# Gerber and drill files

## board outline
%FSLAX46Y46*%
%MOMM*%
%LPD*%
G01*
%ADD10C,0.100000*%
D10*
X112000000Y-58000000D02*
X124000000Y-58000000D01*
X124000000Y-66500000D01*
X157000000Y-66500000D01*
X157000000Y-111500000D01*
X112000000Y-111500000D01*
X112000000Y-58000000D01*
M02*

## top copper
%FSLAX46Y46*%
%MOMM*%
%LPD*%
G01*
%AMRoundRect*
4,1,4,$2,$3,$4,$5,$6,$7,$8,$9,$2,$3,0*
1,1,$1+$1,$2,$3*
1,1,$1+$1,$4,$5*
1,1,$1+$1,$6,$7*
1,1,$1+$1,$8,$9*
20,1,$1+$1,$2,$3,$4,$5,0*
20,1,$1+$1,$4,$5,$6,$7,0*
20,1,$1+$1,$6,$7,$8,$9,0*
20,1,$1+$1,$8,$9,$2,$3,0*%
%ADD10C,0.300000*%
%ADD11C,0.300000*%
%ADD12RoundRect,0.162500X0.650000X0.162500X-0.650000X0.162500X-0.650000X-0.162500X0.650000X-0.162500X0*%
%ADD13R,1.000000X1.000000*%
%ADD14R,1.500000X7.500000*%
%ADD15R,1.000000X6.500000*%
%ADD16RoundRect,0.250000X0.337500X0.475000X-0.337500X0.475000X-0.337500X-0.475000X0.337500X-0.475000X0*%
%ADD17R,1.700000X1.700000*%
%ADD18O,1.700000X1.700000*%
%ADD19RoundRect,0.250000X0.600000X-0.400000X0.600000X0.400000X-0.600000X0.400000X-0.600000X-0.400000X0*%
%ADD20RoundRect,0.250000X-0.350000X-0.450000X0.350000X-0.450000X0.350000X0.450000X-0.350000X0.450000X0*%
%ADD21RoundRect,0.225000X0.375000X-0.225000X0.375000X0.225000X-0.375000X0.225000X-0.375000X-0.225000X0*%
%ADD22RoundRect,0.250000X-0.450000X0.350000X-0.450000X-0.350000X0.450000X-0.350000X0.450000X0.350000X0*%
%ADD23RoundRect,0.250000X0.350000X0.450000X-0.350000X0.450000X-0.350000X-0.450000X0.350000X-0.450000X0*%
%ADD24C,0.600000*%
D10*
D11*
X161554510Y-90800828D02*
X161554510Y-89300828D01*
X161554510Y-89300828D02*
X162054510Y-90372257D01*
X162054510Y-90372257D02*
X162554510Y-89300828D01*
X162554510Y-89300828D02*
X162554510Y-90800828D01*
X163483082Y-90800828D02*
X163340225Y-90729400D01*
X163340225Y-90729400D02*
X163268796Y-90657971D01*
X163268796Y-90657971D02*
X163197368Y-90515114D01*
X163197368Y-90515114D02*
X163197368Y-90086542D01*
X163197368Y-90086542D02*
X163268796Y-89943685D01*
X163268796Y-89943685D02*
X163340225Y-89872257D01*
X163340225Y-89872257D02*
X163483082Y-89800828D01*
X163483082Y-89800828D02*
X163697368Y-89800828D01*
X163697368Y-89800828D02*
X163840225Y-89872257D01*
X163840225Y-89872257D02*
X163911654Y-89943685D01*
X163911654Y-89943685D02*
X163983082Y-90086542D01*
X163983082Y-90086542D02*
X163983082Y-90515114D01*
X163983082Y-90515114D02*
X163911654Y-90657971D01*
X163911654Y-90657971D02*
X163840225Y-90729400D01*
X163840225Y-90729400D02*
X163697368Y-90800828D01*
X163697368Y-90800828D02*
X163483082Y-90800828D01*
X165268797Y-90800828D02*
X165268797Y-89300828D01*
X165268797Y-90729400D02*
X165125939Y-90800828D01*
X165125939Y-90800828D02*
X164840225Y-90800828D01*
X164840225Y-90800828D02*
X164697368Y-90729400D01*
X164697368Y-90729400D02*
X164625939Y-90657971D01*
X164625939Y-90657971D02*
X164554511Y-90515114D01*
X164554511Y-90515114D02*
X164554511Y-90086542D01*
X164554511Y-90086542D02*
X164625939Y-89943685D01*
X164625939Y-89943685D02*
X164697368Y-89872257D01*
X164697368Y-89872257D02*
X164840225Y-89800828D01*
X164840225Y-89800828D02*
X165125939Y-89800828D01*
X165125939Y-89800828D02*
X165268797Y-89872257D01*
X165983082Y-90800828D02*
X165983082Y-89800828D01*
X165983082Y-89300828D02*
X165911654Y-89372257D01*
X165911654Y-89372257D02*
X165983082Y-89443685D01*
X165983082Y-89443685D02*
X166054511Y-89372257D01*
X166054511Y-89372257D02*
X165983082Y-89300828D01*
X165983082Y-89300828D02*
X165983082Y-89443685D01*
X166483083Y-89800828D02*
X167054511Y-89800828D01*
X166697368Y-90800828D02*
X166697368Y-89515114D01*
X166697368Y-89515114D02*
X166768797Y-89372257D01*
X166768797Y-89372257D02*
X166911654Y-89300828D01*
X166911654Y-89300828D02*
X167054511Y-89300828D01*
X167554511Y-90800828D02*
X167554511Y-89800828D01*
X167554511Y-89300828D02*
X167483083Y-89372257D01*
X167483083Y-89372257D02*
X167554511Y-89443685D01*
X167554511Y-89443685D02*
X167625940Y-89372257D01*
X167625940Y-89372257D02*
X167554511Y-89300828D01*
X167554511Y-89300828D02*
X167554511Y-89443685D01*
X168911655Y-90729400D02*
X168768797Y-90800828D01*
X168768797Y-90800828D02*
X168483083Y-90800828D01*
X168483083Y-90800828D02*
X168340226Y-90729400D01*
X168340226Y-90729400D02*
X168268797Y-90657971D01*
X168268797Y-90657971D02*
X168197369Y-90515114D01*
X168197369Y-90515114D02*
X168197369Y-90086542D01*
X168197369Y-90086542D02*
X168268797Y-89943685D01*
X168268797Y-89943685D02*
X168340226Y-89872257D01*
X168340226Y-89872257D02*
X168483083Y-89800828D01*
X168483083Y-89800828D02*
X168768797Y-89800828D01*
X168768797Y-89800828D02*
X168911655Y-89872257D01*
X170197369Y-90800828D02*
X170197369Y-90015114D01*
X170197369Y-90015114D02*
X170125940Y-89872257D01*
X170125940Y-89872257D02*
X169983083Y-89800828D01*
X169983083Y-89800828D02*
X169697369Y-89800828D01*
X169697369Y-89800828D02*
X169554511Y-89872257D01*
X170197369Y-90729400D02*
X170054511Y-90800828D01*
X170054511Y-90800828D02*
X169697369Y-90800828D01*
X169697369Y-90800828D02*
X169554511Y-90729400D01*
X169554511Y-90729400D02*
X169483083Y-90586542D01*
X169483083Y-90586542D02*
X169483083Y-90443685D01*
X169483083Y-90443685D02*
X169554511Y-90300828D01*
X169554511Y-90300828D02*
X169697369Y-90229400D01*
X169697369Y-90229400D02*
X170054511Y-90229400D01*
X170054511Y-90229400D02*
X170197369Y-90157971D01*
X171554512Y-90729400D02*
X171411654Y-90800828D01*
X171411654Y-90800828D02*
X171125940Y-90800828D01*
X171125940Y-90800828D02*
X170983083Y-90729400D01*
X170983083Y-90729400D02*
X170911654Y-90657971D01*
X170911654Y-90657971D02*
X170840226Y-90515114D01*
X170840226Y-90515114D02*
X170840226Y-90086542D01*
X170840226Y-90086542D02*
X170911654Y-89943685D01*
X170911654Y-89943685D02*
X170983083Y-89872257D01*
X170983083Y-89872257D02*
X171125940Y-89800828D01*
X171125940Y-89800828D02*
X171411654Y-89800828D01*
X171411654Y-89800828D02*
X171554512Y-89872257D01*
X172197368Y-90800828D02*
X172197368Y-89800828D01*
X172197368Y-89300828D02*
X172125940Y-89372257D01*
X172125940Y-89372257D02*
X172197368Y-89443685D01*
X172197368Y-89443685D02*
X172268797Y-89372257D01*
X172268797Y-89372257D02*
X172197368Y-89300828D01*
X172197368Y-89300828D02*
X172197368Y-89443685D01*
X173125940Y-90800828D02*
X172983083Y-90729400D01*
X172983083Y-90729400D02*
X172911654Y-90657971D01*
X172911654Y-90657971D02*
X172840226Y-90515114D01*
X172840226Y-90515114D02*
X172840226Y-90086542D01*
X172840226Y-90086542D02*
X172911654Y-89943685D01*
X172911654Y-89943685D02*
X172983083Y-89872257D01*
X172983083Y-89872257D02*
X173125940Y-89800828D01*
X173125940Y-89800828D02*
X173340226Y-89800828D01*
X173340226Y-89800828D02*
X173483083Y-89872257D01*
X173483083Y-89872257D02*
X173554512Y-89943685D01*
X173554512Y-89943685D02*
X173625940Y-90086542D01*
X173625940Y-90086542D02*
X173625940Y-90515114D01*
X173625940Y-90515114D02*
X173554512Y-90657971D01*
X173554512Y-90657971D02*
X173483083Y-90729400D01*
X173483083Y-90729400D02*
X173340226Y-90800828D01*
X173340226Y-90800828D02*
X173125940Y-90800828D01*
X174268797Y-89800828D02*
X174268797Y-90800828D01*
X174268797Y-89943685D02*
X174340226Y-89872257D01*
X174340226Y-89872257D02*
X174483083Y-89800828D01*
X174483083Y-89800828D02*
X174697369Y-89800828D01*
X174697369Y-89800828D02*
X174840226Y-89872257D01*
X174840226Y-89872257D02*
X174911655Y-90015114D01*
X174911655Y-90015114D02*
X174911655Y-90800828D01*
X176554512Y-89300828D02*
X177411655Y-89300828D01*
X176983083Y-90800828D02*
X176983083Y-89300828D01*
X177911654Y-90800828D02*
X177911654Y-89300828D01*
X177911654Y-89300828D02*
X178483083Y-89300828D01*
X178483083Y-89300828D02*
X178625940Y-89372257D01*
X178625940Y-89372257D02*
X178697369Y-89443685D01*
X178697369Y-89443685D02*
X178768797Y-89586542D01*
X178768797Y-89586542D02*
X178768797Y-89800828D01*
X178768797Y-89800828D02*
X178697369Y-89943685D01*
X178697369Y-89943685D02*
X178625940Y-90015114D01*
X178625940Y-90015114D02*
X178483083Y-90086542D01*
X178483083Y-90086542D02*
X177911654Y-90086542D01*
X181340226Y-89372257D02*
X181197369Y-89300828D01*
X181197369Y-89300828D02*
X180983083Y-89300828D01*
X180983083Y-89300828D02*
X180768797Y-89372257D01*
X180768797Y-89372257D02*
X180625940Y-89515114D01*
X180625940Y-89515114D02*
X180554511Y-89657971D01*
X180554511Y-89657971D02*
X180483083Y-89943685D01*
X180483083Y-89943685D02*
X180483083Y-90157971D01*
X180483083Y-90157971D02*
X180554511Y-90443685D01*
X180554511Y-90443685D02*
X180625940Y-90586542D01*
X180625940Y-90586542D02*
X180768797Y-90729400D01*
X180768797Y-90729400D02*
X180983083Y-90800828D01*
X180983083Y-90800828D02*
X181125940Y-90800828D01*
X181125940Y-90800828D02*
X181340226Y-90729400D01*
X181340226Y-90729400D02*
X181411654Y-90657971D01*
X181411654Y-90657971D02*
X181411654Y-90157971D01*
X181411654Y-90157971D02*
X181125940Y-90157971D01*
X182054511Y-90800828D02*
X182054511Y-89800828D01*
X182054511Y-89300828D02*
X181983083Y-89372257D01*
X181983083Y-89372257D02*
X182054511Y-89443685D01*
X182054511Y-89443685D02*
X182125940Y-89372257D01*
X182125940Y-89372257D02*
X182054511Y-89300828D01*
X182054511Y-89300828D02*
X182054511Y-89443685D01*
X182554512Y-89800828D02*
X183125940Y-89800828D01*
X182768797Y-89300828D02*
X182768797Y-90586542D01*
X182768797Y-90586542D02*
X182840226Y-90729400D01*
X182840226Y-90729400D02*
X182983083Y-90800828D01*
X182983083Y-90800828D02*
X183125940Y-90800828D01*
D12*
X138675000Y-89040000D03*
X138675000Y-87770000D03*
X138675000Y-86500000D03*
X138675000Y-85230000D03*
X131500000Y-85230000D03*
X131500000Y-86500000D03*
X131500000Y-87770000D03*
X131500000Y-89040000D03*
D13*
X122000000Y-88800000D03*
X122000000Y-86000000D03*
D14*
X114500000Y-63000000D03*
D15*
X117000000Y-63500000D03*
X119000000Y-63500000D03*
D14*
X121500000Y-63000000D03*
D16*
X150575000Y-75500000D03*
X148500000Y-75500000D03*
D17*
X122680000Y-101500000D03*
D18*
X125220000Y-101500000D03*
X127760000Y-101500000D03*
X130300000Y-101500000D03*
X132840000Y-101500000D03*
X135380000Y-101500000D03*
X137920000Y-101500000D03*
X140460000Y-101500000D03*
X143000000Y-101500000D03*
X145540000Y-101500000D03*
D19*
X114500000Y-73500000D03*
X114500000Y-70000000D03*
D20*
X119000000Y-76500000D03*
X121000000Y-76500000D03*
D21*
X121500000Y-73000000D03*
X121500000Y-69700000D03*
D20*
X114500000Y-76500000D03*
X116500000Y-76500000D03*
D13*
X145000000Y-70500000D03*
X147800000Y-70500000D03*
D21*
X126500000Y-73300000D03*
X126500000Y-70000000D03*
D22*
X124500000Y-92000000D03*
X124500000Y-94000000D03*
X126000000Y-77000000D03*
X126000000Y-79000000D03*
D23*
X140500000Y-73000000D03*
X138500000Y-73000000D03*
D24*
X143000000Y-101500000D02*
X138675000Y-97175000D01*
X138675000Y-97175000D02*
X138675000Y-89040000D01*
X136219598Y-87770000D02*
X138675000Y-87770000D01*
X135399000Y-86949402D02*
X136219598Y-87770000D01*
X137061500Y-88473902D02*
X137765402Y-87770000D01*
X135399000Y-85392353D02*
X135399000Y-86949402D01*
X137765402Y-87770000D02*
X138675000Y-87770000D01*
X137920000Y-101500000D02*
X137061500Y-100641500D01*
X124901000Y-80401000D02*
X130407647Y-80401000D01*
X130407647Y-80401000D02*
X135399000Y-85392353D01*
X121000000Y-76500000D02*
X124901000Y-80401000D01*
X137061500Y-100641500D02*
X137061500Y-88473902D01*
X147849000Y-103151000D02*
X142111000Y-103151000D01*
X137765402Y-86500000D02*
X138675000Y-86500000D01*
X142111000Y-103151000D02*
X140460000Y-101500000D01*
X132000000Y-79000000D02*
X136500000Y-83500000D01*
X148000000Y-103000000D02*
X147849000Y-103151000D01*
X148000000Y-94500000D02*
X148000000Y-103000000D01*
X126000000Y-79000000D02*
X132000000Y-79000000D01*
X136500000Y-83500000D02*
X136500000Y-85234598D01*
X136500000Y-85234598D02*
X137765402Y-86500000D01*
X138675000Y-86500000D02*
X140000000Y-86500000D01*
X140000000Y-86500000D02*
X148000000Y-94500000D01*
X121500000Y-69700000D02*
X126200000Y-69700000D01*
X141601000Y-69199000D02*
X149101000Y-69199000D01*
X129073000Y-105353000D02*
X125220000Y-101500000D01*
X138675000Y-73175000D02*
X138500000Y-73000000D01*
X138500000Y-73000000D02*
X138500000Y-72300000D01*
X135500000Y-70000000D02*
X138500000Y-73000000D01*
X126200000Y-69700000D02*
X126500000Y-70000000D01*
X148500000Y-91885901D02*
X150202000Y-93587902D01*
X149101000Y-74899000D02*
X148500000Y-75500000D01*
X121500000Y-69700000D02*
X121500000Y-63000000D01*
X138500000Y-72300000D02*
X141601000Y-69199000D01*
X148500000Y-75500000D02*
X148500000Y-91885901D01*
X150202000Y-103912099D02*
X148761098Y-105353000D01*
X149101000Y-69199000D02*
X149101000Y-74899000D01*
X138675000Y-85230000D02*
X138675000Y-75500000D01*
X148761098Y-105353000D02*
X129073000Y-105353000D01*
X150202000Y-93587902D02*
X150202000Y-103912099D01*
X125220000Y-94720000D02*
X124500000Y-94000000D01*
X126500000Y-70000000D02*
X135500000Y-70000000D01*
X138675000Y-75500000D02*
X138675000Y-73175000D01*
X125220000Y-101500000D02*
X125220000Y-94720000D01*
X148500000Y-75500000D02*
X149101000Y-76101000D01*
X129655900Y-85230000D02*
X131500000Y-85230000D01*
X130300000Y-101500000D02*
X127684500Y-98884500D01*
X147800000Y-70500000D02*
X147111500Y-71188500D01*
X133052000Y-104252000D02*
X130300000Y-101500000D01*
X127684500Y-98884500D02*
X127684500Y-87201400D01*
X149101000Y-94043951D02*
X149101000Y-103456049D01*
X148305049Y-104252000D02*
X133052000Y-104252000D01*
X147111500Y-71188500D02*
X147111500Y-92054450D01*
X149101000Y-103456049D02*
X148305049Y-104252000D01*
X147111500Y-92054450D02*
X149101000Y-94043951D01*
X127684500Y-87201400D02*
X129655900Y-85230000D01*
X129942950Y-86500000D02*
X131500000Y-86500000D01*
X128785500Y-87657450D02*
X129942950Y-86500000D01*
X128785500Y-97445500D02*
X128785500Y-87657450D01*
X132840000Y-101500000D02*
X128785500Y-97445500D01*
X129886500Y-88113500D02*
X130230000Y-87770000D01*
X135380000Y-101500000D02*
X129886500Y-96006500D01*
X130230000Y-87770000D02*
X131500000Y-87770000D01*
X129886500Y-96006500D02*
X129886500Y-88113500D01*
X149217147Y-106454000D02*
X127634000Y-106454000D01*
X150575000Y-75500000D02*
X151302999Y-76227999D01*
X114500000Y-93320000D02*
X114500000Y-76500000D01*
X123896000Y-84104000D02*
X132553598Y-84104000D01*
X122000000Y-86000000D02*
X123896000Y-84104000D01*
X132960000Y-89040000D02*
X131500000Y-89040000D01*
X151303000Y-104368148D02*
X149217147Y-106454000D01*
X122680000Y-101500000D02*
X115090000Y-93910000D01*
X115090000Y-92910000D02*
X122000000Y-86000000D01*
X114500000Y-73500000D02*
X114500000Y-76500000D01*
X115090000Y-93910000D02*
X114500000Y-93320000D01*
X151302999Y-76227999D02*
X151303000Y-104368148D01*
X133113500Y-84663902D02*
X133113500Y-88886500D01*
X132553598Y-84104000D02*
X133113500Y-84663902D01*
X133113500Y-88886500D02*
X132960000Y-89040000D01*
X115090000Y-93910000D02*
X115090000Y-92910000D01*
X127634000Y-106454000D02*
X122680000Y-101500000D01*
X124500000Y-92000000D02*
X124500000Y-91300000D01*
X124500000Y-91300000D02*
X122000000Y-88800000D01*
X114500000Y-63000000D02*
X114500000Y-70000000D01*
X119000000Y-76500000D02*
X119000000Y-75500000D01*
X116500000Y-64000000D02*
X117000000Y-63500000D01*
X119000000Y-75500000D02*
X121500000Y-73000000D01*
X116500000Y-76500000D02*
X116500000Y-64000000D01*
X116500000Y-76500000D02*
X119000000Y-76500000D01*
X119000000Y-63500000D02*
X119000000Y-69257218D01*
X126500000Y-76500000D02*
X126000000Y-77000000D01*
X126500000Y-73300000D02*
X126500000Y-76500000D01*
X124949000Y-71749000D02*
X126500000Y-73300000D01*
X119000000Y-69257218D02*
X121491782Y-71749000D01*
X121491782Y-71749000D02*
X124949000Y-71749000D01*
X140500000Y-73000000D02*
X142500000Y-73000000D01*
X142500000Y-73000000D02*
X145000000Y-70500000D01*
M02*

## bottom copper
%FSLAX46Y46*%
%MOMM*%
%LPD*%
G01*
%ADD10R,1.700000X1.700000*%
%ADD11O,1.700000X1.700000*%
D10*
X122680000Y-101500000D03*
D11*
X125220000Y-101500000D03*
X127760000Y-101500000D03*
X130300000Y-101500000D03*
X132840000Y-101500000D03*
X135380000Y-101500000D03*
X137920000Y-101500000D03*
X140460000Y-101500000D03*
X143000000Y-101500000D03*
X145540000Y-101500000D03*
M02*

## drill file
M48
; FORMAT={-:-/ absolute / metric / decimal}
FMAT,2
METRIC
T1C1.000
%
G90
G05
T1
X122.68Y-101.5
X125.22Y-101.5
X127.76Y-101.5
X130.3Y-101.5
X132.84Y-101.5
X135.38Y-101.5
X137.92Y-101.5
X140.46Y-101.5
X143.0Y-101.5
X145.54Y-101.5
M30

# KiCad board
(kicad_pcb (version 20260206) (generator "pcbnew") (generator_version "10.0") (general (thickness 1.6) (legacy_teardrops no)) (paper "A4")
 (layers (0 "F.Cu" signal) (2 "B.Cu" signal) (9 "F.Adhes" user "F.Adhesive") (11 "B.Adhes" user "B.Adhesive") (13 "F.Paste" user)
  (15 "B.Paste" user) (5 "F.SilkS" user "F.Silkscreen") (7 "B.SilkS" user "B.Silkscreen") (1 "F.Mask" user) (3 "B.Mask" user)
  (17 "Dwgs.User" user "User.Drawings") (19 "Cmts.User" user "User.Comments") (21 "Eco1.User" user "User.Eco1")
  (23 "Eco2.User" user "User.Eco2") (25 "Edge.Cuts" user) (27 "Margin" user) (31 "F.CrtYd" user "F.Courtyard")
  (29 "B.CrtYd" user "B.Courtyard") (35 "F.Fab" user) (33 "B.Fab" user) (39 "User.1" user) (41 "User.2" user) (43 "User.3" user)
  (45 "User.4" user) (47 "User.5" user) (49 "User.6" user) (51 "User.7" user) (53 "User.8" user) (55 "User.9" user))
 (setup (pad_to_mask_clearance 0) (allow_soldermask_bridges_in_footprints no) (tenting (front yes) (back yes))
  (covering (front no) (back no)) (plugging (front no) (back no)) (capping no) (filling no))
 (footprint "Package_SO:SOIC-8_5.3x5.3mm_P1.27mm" (layer "F.Cu") (at 135.0875 87.135 180)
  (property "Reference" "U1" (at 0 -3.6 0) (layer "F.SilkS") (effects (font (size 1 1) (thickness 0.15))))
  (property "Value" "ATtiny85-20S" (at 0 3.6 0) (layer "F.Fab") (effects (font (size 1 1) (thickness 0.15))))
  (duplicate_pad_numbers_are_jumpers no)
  (pad "1" smd roundrect (at -3.5875 -1.905 180) (size 1.625 0.65) (layers "F.Cu" "F.Mask" "F.Paste") (roundrect_rratio 0.25)
   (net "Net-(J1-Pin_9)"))
  (pad "2" smd roundrect (at -3.5875 -0.635 180) (size 1.625 0.65) (layers "F.Cu" "F.Mask" "F.Paste") (roundrect_rratio 0.25)
   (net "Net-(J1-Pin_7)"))
  (pad "3" smd roundrect (at -3.5875 0.635 180) (size 1.625 0.65) (layers "F.Cu" "F.Mask" "F.Paste") (roundrect_rratio 0.25)
   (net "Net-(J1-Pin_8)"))
  (pad "4" smd roundrect (at -3.5875 1.905 180) (size 1.625 0.65) (layers "F.Cu" "F.Mask" "F.Paste") (roundrect_rratio 0.25) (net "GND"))
  (pad "5" smd roundrect (at 3.5875 1.905 180) (size 1.625 0.65) (layers "F.Cu" "F.Mask" "F.Paste") (roundrect_rratio 0.25)
   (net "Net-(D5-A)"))
  (pad "6" smd roundrect (at 3.5875 0.635 180) (size 1.625 0.65) (layers "F.Cu" "F.Mask" "F.Paste") (roundrect_rratio 0.25)
   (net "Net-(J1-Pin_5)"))
  (pad "7" smd roundrect (at 3.5875 -0.635 180) (size 1.625 0.65) (layers "F.Cu" "F.Mask" "F.Paste") (roundrect_rratio 0.25)
   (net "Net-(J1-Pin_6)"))
  (pad "8" smd roundrect (at 3.5875 -1.905 180) (size 1.625 0.65) (layers "F.Cu" "F.Mask" "F.Paste") (roundrect_rratio 0.25) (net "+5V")))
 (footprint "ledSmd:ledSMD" (layer "F.Cu") (at 122 87 90)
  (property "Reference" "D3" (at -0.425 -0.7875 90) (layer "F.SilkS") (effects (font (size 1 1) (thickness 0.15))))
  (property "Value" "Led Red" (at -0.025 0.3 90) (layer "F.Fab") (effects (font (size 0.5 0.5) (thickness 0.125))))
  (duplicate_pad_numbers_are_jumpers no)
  (pad "1" smd rect (at -1.8 0 90) (size 1 1) (layers "F.Cu" "F.Mask" "F.Paste") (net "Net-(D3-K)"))
  (pad "2" smd rect (at 1 0 90) (size 1 1) (layers "F.Cu" "F.Mask" "F.Paste") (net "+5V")))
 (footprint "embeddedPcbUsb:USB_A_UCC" (layer "F.Cu") (at 118 63.2 -90)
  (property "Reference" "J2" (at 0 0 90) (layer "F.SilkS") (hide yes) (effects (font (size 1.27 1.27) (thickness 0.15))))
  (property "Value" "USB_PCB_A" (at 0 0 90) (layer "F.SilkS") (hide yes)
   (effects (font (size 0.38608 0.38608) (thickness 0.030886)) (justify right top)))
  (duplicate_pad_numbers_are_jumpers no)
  (pad "1" smd rect (at -0.2 3.5 270) (size 7.5 1.5) (layers "F.Cu" "F.Mask" "F.Paste") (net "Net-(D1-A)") (solder_mask_margin 0.1016))
  (pad "2" smd rect (at 0.3 1 270) (size 6.5 1) (layers "F.Cu" "F.Mask" "F.Paste") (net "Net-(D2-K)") (solder_mask_margin 0.1016))
  (pad "3" smd rect (at 0.3 -1 270) (size 6.5 1) (layers "F.Cu" "F.Mask" "F.Paste") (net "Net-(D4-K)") (solder_mask_margin 0.1016))
  (pad "4" smd rect (at -0.2 -3.5 270) (size 7.5 1.5) (layers "F.Cu" "F.Mask" "F.Paste") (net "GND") (solder_mask_margin 0.1016)))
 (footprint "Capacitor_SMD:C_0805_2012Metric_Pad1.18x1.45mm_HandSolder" (layer "F.Cu") (at 149.5375 75.5 180)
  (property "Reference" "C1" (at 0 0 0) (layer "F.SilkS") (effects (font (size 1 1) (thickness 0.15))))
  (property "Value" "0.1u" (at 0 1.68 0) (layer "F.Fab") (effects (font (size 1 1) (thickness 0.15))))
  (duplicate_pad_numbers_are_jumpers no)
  (pad "1" smd roundrect (at -1.0375 0 180) (size 1.175 1.45) (layers "F.Cu" "F.Mask" "F.Paste") (roundrect_rratio 0.212766) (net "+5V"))
  (pad "2" smd roundrect (at 1.0375 0 180) (size 1.175 1.45) (layers "F.Cu" "F.Mask" "F.Paste") (roundrect_rratio 0.212766) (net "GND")))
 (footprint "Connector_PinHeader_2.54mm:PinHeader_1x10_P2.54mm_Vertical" (layer "F.Cu") (at 122.68 101.5 90)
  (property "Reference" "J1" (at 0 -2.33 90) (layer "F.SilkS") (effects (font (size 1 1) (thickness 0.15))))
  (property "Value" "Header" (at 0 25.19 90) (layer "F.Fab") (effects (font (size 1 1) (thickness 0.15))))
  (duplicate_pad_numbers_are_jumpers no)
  (pad "1" thru_hole rect (at 0 0 90) (size 1.7 1.7) (drill 1) (layers "*.Cu" "*.Mask") (remove_unused_layers no) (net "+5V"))
  (pad "2" thru_hole oval (at 0 2.54 90) (size 1.7 1.7) (drill 1) (layers "*.Cu" "*.Mask") (remove_unused_layers no) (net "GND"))
  (pad "3" thru_hole oval (at 0 5.08 90) (size 1.7 1.7) (drill 1) (layers "*.Cu" "*.Mask") (remove_unused_layers no)
   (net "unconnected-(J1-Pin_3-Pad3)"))
  (pad "4" thru_hole oval (at 0 7.62 90) (size 1.7 1.7) (drill 1) (layers "*.Cu" "*.Mask") (remove_unused_layers no) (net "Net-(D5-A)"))
  (pad "5" thru_hole oval (at 0 10.16 90) (size 1.7 1.7) (drill 1) (layers "*.Cu" "*.Mask") (remove_unused_layers no) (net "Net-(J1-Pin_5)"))
  (pad "6" thru_hole oval (at 0 12.7 90) (size 1.7 1.7) (drill 1) (layers "*.Cu" "*.Mask") (remove_unused_layers no) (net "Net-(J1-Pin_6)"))
  (pad "7" thru_hole oval (at 0 15.24 90) (size 1.7 1.7) (drill 1) (layers "*.Cu" "*.Mask") (remove_unused_layers no) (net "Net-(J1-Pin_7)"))
  (pad "8" thru_hole oval (at 0 17.78 90) (size 1.7 1.7) (drill 1) (layers "*.Cu" "*.Mask") (remove_unused_layers no) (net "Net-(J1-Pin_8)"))
  (pad "9" thru_hole oval (at 0 20.32 90) (size 1.7 1.7) (drill 1) (layers "*.Cu" "*.Mask") (remove_unused_layers no) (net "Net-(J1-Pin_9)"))
  (pad "10" thru_hole oval (at 0 22.86 90) (size 1.7 1.7) (drill 1) (layers "*.Cu" "*.Mask") (remove_unused_layers no)
   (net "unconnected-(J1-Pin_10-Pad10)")))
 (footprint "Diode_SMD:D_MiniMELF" (layer "F.Cu") (at 114.5 71.75 90)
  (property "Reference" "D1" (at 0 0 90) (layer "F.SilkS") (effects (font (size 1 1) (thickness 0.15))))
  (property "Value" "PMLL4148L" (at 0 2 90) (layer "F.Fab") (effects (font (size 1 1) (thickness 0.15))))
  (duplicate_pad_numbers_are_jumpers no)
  (pad "1" smd roundrect (at -1.75 0 90) (size 1.3 1.7) (layers "F.Cu" "F.Mask" "F.Paste") (roundrect_rratio 0.1923076923) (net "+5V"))
  (pad "2" smd roundrect (at 1.75 0 90) (size 1.3 1.7) (layers "F.Cu" "F.Mask" "F.Paste") (roundrect_rratio 0.1923076923) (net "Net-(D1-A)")))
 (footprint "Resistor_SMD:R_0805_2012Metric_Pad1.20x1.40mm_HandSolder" (layer "F.Cu") (at 120 76.5)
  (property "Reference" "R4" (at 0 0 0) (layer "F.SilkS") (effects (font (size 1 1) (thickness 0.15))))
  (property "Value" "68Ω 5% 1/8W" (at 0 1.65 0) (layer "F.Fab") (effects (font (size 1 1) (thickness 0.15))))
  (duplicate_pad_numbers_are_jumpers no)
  (pad "1" smd roundrect (at -1 0) (size 1.2 1.4) (layers "F.Cu" "F.Mask" "F.Paste") (roundrect_rratio 0.208333) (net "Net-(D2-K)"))
  (pad "2" smd roundrect (at 1 0) (size 1.2 1.4) (layers "F.Cu" "F.Mask" "F.Paste") (roundrect_rratio 0.208333) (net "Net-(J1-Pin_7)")))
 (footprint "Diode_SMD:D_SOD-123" (layer "F.Cu") (at 121.5 71.35 90)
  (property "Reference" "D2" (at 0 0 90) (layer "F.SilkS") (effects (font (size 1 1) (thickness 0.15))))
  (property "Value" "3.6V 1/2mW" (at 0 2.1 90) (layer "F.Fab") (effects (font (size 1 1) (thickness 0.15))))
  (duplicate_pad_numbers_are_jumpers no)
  (pad "1" smd roundrect (at -1.65 0 90) (size 0.9 1.2) (layers "F.Cu" "F.Mask" "F.Paste") (roundrect_rratio 0.25) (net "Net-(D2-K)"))
  (pad "2" smd roundrect (at 1.65 0 90) (size 0.9 1.2) (layers "F.Cu" "F.Mask" "F.Paste") (roundrect_rratio 0.25) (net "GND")))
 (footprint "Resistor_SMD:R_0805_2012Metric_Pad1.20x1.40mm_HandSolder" (layer "F.Cu") (at 115.5 76.5)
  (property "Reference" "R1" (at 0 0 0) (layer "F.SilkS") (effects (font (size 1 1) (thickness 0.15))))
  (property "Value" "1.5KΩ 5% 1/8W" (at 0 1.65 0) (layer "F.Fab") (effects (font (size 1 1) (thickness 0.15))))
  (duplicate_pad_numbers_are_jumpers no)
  (pad "1" smd roundrect (at -1 0) (size 1.2 1.4) (layers "F.Cu" "F.Mask" "F.Paste") (roundrect_rratio 0.208333) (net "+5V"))
  (pad "2" smd roundrect (at 1 0) (size 1.2 1.4) (layers "F.Cu" "F.Mask" "F.Paste") (roundrect_rratio 0.208333) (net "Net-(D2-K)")))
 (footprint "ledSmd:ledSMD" (layer "F.Cu") (at 146.8 70.5)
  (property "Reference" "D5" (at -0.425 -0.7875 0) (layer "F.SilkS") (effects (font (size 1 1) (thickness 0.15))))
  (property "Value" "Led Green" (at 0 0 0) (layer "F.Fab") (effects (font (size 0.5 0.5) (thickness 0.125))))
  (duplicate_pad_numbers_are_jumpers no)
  (pad "1" smd rect (at -1.8 0) (size 1 1) (layers "F.Cu" "F.Mask" "F.Paste") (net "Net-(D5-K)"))
  (pad "2" smd rect (at 1 0) (size 1 1) (layers "F.Cu" "F.Mask" "F.Paste") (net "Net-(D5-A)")))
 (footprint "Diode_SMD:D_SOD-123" (layer "F.Cu") (at 126.5 71.65 90)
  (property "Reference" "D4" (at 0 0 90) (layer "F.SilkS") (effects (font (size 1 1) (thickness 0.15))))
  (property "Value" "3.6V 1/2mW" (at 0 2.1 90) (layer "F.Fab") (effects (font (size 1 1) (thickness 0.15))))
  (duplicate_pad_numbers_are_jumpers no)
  (pad "1" smd roundrect (at -1.65 0 90) (size 0.9 1.2) (layers "F.Cu" "F.Mask" "F.Paste") (roundrect_rratio 0.25) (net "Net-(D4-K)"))
  (pad "2" smd roundrect (at 1.65 0 90) (size 0.9 1.2) (layers "F.Cu" "F.Mask" "F.Paste") (roundrect_rratio 0.25) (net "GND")))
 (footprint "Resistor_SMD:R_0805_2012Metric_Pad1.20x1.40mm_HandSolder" (layer "F.Cu") (at 124.5 93 -90)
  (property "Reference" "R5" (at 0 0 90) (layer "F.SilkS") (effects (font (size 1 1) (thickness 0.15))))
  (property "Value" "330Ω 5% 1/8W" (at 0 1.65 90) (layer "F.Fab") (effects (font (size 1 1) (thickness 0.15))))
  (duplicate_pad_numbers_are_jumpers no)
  (pad "1" smd roundrect (at -1 0 270) (size 1.2 1.4) (layers "F.Cu" "F.Mask" "F.Paste") (roundrect_rratio 0.208333) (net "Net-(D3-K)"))
  (pad "2" smd roundrect (at 1 0 270) (size 1.2 1.4) (layers "F.Cu" "F.Mask" "F.Paste") (roundrect_rratio 0.208333) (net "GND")))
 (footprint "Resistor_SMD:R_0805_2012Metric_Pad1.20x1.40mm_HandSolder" (layer "F.Cu") (at 126 78 -90)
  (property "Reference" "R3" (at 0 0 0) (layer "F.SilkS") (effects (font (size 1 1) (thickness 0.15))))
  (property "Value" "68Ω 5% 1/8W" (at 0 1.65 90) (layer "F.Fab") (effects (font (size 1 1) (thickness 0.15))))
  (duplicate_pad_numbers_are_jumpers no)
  (pad "1" smd roundrect (at -1 0 270) (size 1.2 1.4) (layers "F.Cu" "F.Mask" "F.Paste") (roundrect_rratio 0.208333) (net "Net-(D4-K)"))
  (pad "2" smd roundrect (at 1 0 270) (size 1.2 1.4) (layers "F.Cu" "F.Mask" "F.Paste") (roundrect_rratio 0.208333) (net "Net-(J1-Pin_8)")))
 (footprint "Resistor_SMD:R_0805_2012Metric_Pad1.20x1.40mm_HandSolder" (layer "F.Cu") (at 139.5 73 180)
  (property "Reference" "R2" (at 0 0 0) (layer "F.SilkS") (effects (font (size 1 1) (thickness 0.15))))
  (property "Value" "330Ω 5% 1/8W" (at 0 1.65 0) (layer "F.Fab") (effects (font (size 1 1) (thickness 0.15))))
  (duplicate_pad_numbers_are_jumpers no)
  (pad "1" smd roundrect (at -1 0 180) (size 1.2 1.4) (layers "F.Cu" "F.Mask" "F.Paste") (roundrect_rratio 0.208333) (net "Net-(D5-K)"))
  (pad "2" smd roundrect (at 1 0 180) (size 1.2 1.4) (layers "F.Cu" "F.Mask" "F.Paste") (roundrect_rratio 0.208333) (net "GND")))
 (gr_poly
  (pts (xy 112 58) (xy 124 58) (xy 124 66.5) (xy 157 66.5) (xy 157 111.5) (xy 112 111.5)) (stroke (width 0.1) (type solid)) (fill no)
  (layer "Edge.Cuts"))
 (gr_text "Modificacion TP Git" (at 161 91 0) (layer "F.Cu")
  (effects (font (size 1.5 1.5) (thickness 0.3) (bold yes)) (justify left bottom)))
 (segment (start 143 101.5) (end 138.675 97.175) (width 0.6) (layer "F.Cu") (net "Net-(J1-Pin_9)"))
 (segment (start 138.675 97.175) (end 138.675 89.04) (width 0.6) (layer "F.Cu") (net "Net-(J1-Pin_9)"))
 (segment (start 136.219598 87.77) (end 138.675 87.77) (width 0.6) (layer "F.Cu") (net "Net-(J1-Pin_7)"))
 (segment (start 135.399 86.949402) (end 136.219598 87.77) (width 0.6) (layer "F.Cu") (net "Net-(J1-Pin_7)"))
 (segment (start 137.0615 88.473902) (end 137.765402 87.77) (width 0.6) (layer "F.Cu") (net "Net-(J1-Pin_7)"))
 (segment (start 135.399 85.392353) (end 135.399 86.949402) (width 0.6) (layer "F.Cu") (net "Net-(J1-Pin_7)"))
 (segment (start 137.765402 87.77) (end 138.675 87.77) (width 0.6) (layer "F.Cu") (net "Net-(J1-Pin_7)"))
 (segment (start 137.92 101.5) (end 137.0615 100.6415) (width 0.6) (layer "F.Cu") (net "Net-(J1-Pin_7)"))
 (segment (start 124.901 80.401) (end 130.407647 80.401) (width 0.6) (layer "F.Cu") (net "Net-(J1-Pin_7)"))
 (segment (start 130.407647 80.401) (end 135.399 85.392353) (width 0.6) (layer "F.Cu") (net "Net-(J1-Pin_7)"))
 (segment (start 121 76.5) (end 124.901 80.401) (width 0.6) (layer "F.Cu") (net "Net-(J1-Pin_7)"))
 (segment (start 137.0615 100.6415) (end 137.0615 88.473902) (width 0.6) (layer "F.Cu") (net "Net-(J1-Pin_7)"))
 (segment (start 147.849 103.151) (end 142.111 103.151) (width 0.6) (layer "F.Cu") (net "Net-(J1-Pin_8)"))
 (segment (start 137.765402 86.5) (end 138.675 86.5) (width 0.6) (layer "F.Cu") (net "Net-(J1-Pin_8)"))
 (segment (start 142.111 103.151) (end 140.46 101.5) (width 0.6) (layer "F.Cu") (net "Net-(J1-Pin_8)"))
 (segment (start 132 79) (end 136.5 83.5) (width 0.6) (layer "F.Cu") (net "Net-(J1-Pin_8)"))
 (segment (start 148 103) (end 147.849 103.151) (width 0.6) (layer "F.Cu") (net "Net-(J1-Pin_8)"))
 (segment (start 148 94.5) (end 148 103) (width 0.6) (layer "F.Cu") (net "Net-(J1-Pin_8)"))
 (segment (start 126 79) (end 132 79) (width 0.6) (layer "F.Cu") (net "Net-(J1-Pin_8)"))
 (segment (start 136.5 83.5) (end 136.5 85.234598) (width 0.6) (layer "F.Cu") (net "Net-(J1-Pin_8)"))
 (segment (start 136.5 85.234598) (end 137.765402 86.5) (width 0.6) (layer "F.Cu") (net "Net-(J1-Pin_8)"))
 (segment (start 138.675 86.5) (end 140 86.5) (width 0.6) (layer "F.Cu") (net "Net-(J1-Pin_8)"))
 (segment (start 140 86.5) (end 148 94.5) (width 0.6) (layer "F.Cu") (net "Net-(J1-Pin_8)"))
 (segment (start 121.5 69.7) (end 126.2 69.7) (width 0.6) (layer "F.Cu") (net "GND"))
 (segment (start 141.601 69.199) (end 149.101 69.199) (width 0.6) (layer "F.Cu") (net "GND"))
 (segment (start 129.073 105.353) (end 125.22 101.5) (width 0.6) (layer "F.Cu") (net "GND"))
 (segment (start 138.675 73.175) (end 138.5 73) (width 0.6) (layer "F.Cu") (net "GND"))
 (segment (start 138.5 73) (end 138.5 72.3) (width 0.6) (layer "F.Cu") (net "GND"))
 (segment (start 135.5 70) (end 138.5 73) (width 0.6) (layer "F.Cu") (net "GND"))
 (segment (start 126.2 69.7) (end 126.5 70) (width 0.6) (layer "F.Cu") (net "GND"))
 (segment (start 148.5 91.885901) (end 150.202 93.587902) (width 0.6) (layer "F.Cu") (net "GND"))
 (segment (start 149.101 74.899) (end 148.5 75.5) (width 0.6) (layer "F.Cu") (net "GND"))
 (segment (start 121.5 69.7) (end 121.5 63) (width 0.6) (layer "F.Cu") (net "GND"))
 (segment (start 138.5 72.3) (end 141.601 69.199) (width 0.6) (layer "F.Cu") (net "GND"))
 (segment (start 148.5 75.5) (end 148.5 91.885901) (width 0.6) (layer "F.Cu") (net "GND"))
 (segment (start 150.202 103.912099) (end 148.761098 105.353) (width 0.6) (layer "F.Cu") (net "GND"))
 (segment (start 149.101 69.199) (end 149.101 74.899) (width 0.6) (layer "F.Cu") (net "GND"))
 (segment (start 138.675 85.23) (end 138.675 75.5) (width 0.6) (layer "F.Cu") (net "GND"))
 (segment (start 148.761098 105.353) (end 129.073 105.353) (width 0.6) (layer "F.Cu") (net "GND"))
 (segment (start 150.202 93.587902) (end 150.202 103.912099) (width 0.6) (layer "F.Cu") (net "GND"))
 (segment (start 125.22 94.72) (end 124.5 94) (width 0.6) (layer "F.Cu") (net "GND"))
 (segment (start 126.5 70) (end 135.5 70) (width 0.6) (layer "F.Cu") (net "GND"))
 (segment (start 138.675 75.5) (end 138.675 73.175) (width 0.6) (layer "F.Cu") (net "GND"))
 (segment (start 125.22 101.5) (end 125.22 94.72) (width 0.6) (layer "F.Cu") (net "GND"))
 (segment (start 148.5 75.5) (end 149.101 76.101) (width 0.6) (layer "F.Cu") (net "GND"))
 (segment (start 129.6559 85.23) (end 131.5 85.23) (width 0.6) (layer "F.Cu") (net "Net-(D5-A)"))
 (segment (start 130.3 101.5) (end 127.6845 98.8845) (width 0.6) (layer "F.Cu") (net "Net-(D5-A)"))
 (segment (start 147.8 70.5) (end 147.1115 71.1885) (width 0.6) (layer "F.Cu") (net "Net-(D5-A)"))
 (segment (start 133.052 104.252) (end 130.3 101.5) (width 0.6) (layer "F.Cu") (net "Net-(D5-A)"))
 (segment (start 127.6845 98.8845) (end 127.6845 87.2014) (width 0.6) (layer "F.Cu") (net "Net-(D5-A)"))
 (segment (start 149.101 94.043951) (end 149.101 103.456049) (width 0.6) (layer "F.Cu") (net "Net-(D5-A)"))
 (segment (start 148.305049 104.252) (end 133.052 104.252) (width 0.6) (layer "F.Cu") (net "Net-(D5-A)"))
 (segment (start 147.1115 71.1885) (end 147.1115 92.05445) (width 0.6) (layer "F.Cu") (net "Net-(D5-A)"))
 (segment (start 149.101 103.456049) (end 148.305049 104.252) (width 0.6) (layer "F.Cu") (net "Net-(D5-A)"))
 (segment (start 147.1115 92.05445) (end 149.101 94.043951) (width 0.6) (layer "F.Cu") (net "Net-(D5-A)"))
 (segment (start 127.6845 87.2014) (end 129.6559 85.23) (width 0.6) (layer "F.Cu") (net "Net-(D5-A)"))
 (segment (start 129.94295 86.5) (end 131.5 86.5) (width 0.6) (layer "F.Cu") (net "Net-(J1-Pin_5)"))
 (segment (start 128.7855 87.65745) (end 129.94295 86.5) (width 0.6) (layer "F.Cu") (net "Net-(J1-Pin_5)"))
 (segment (start 128.7855 97.4455) (end 128.7855 87.65745) (width 0.6) (layer "F.Cu") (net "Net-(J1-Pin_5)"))
 (segment (start 132.84 101.5) (end 128.7855 97.4455) (width 0.6) (layer "F.Cu") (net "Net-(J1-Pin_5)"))
 (segment (start 129.8865 88.1135) (end 130.23 87.77) (width 0.6) (layer "F.Cu") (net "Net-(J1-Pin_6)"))
 (segment (start 135.38 101.5) (end 129.8865 96.0065) (width 0.6) (layer "F.Cu") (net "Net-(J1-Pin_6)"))
 (segment (start 130.23 87.77) (end 131.5 87.77) (width 0.6) (layer "F.Cu") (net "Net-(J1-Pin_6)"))
 (segment (start 129.8865 96.0065) (end 129.8865 88.1135) (width 0.6) (layer "F.Cu") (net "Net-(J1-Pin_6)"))
 (segment (start 149.217147 106.454) (end 127.634 106.454) (width 0.6) (layer "F.Cu") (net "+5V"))
 (segment (start 150.575 75.5) (end 151.302999 76.227999) (width 0.6) (layer "F.Cu") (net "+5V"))
 (segment (start 114.5 93.32) (end 114.5 76.5) (width 0.6) (layer "F.Cu") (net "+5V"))
 (segment (start 123.896 84.104) (end 132.553598 84.104) (width 0.6) (layer "F.Cu") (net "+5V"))
 (segment (start 122 86) (end 123.896 84.104) (width 0.6) (layer "F.Cu") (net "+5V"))
 (segment (start 132.96 89.04) (end 131.5 89.04) (width 0.6) (layer "F.Cu") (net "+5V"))
 (segment (start 151.303 104.368148) (end 149.217147 106.454) (width 0.6) (layer "F.Cu") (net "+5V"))
 (segment (start 122.68 101.5) (end 115.09 93.91) (width 0.6) (layer "F.Cu") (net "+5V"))
 (segment (start 115.09 92.91) (end 122 86) (width 0.6) (layer "F.Cu") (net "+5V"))
 (segment (start 114.5 73.5) (end 114.5 76.5) (width 0.6) (layer "F.Cu") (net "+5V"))
 (segment (start 115.09 93.91) (end 114.5 93.32) (width 0.6) (layer "F.Cu") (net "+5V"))
 (segment (start 151.302999 76.227999) (end 151.303 104.368148) (width 0.6) (layer "F.Cu") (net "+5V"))
 (segment (start 133.1135 84.663902) (end 133.1135 88.8865) (width 0.6) (layer "F.Cu") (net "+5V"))
 (segment (start 132.553598 84.104) (end 133.1135 84.663902) (width 0.6) (layer "F.Cu") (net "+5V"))
 (segment (start 133.1135 88.8865) (end 132.96 89.04) (width 0.6) (layer "F.Cu") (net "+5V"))
 (segment (start 115.09 93.91) (end 115.09 92.91) (width 0.6) (layer "F.Cu") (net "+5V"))
 (segment (start 127.634 106.454) (end 122.68 101.5) (width 0.6) (layer "F.Cu") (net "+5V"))
 (segment (start 124.5 92) (end 124.5 91.3) (width 0.6) (layer "F.Cu") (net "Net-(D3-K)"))
 (segment (start 124.5 91.3) (end 122 88.8) (width 0.6) (layer "F.Cu") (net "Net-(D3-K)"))
 (segment (start 114.5 63) (end 114.5 70) (width 0.6) (layer "F.Cu") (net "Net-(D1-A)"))
 (segment (start 119 76.5) (end 119 75.5) (width 0.6) (layer "F.Cu") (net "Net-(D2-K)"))
 (segment (start 116.5 64) (end 117 63.5) (width 0.6) (layer "F.Cu") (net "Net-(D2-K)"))
 (segment (start 119 75.5) (end 121.5 73) (width 0.6) (layer "F.Cu") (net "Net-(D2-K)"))
 (segment (start 116.5 76.5) (end 116.5 64) (width 0.6) (layer "F.Cu") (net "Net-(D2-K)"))
 (segment (start 116.5 76.5) (end 119 76.5) (width 0.6) (layer "F.Cu") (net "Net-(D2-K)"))
 (segment (start 119 63.5) (end 119 69.257218) (width 0.6) (layer "F.Cu") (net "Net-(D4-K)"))
 (segment (start 126.5 76.5) (end 126 77) (width 0.6) (layer "F.Cu") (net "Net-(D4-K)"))
 (segment (start 126.5 73.3) (end 126.5 76.5) (width 0.6) (layer "F.Cu") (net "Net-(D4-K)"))
 (segment (start 124.949 71.749) (end 126.5 73.3) (width 0.6) (layer "F.Cu") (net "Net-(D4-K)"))
 (segment (start 119 69.257218) (end 121.491782 71.749) (width 0.6) (layer "F.Cu") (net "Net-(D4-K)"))
 (segment (start 121.491782 71.749) (end 124.949 71.749) (width 0.6) (layer "F.Cu") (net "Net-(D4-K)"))
 (segment (start 140.5 73) (end 142.5 73) (width 0.6) (layer "F.Cu") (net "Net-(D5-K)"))
 (segment (start 142.5 73) (end 145 70.5) (width 0.6) (layer "F.Cu") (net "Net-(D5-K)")))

